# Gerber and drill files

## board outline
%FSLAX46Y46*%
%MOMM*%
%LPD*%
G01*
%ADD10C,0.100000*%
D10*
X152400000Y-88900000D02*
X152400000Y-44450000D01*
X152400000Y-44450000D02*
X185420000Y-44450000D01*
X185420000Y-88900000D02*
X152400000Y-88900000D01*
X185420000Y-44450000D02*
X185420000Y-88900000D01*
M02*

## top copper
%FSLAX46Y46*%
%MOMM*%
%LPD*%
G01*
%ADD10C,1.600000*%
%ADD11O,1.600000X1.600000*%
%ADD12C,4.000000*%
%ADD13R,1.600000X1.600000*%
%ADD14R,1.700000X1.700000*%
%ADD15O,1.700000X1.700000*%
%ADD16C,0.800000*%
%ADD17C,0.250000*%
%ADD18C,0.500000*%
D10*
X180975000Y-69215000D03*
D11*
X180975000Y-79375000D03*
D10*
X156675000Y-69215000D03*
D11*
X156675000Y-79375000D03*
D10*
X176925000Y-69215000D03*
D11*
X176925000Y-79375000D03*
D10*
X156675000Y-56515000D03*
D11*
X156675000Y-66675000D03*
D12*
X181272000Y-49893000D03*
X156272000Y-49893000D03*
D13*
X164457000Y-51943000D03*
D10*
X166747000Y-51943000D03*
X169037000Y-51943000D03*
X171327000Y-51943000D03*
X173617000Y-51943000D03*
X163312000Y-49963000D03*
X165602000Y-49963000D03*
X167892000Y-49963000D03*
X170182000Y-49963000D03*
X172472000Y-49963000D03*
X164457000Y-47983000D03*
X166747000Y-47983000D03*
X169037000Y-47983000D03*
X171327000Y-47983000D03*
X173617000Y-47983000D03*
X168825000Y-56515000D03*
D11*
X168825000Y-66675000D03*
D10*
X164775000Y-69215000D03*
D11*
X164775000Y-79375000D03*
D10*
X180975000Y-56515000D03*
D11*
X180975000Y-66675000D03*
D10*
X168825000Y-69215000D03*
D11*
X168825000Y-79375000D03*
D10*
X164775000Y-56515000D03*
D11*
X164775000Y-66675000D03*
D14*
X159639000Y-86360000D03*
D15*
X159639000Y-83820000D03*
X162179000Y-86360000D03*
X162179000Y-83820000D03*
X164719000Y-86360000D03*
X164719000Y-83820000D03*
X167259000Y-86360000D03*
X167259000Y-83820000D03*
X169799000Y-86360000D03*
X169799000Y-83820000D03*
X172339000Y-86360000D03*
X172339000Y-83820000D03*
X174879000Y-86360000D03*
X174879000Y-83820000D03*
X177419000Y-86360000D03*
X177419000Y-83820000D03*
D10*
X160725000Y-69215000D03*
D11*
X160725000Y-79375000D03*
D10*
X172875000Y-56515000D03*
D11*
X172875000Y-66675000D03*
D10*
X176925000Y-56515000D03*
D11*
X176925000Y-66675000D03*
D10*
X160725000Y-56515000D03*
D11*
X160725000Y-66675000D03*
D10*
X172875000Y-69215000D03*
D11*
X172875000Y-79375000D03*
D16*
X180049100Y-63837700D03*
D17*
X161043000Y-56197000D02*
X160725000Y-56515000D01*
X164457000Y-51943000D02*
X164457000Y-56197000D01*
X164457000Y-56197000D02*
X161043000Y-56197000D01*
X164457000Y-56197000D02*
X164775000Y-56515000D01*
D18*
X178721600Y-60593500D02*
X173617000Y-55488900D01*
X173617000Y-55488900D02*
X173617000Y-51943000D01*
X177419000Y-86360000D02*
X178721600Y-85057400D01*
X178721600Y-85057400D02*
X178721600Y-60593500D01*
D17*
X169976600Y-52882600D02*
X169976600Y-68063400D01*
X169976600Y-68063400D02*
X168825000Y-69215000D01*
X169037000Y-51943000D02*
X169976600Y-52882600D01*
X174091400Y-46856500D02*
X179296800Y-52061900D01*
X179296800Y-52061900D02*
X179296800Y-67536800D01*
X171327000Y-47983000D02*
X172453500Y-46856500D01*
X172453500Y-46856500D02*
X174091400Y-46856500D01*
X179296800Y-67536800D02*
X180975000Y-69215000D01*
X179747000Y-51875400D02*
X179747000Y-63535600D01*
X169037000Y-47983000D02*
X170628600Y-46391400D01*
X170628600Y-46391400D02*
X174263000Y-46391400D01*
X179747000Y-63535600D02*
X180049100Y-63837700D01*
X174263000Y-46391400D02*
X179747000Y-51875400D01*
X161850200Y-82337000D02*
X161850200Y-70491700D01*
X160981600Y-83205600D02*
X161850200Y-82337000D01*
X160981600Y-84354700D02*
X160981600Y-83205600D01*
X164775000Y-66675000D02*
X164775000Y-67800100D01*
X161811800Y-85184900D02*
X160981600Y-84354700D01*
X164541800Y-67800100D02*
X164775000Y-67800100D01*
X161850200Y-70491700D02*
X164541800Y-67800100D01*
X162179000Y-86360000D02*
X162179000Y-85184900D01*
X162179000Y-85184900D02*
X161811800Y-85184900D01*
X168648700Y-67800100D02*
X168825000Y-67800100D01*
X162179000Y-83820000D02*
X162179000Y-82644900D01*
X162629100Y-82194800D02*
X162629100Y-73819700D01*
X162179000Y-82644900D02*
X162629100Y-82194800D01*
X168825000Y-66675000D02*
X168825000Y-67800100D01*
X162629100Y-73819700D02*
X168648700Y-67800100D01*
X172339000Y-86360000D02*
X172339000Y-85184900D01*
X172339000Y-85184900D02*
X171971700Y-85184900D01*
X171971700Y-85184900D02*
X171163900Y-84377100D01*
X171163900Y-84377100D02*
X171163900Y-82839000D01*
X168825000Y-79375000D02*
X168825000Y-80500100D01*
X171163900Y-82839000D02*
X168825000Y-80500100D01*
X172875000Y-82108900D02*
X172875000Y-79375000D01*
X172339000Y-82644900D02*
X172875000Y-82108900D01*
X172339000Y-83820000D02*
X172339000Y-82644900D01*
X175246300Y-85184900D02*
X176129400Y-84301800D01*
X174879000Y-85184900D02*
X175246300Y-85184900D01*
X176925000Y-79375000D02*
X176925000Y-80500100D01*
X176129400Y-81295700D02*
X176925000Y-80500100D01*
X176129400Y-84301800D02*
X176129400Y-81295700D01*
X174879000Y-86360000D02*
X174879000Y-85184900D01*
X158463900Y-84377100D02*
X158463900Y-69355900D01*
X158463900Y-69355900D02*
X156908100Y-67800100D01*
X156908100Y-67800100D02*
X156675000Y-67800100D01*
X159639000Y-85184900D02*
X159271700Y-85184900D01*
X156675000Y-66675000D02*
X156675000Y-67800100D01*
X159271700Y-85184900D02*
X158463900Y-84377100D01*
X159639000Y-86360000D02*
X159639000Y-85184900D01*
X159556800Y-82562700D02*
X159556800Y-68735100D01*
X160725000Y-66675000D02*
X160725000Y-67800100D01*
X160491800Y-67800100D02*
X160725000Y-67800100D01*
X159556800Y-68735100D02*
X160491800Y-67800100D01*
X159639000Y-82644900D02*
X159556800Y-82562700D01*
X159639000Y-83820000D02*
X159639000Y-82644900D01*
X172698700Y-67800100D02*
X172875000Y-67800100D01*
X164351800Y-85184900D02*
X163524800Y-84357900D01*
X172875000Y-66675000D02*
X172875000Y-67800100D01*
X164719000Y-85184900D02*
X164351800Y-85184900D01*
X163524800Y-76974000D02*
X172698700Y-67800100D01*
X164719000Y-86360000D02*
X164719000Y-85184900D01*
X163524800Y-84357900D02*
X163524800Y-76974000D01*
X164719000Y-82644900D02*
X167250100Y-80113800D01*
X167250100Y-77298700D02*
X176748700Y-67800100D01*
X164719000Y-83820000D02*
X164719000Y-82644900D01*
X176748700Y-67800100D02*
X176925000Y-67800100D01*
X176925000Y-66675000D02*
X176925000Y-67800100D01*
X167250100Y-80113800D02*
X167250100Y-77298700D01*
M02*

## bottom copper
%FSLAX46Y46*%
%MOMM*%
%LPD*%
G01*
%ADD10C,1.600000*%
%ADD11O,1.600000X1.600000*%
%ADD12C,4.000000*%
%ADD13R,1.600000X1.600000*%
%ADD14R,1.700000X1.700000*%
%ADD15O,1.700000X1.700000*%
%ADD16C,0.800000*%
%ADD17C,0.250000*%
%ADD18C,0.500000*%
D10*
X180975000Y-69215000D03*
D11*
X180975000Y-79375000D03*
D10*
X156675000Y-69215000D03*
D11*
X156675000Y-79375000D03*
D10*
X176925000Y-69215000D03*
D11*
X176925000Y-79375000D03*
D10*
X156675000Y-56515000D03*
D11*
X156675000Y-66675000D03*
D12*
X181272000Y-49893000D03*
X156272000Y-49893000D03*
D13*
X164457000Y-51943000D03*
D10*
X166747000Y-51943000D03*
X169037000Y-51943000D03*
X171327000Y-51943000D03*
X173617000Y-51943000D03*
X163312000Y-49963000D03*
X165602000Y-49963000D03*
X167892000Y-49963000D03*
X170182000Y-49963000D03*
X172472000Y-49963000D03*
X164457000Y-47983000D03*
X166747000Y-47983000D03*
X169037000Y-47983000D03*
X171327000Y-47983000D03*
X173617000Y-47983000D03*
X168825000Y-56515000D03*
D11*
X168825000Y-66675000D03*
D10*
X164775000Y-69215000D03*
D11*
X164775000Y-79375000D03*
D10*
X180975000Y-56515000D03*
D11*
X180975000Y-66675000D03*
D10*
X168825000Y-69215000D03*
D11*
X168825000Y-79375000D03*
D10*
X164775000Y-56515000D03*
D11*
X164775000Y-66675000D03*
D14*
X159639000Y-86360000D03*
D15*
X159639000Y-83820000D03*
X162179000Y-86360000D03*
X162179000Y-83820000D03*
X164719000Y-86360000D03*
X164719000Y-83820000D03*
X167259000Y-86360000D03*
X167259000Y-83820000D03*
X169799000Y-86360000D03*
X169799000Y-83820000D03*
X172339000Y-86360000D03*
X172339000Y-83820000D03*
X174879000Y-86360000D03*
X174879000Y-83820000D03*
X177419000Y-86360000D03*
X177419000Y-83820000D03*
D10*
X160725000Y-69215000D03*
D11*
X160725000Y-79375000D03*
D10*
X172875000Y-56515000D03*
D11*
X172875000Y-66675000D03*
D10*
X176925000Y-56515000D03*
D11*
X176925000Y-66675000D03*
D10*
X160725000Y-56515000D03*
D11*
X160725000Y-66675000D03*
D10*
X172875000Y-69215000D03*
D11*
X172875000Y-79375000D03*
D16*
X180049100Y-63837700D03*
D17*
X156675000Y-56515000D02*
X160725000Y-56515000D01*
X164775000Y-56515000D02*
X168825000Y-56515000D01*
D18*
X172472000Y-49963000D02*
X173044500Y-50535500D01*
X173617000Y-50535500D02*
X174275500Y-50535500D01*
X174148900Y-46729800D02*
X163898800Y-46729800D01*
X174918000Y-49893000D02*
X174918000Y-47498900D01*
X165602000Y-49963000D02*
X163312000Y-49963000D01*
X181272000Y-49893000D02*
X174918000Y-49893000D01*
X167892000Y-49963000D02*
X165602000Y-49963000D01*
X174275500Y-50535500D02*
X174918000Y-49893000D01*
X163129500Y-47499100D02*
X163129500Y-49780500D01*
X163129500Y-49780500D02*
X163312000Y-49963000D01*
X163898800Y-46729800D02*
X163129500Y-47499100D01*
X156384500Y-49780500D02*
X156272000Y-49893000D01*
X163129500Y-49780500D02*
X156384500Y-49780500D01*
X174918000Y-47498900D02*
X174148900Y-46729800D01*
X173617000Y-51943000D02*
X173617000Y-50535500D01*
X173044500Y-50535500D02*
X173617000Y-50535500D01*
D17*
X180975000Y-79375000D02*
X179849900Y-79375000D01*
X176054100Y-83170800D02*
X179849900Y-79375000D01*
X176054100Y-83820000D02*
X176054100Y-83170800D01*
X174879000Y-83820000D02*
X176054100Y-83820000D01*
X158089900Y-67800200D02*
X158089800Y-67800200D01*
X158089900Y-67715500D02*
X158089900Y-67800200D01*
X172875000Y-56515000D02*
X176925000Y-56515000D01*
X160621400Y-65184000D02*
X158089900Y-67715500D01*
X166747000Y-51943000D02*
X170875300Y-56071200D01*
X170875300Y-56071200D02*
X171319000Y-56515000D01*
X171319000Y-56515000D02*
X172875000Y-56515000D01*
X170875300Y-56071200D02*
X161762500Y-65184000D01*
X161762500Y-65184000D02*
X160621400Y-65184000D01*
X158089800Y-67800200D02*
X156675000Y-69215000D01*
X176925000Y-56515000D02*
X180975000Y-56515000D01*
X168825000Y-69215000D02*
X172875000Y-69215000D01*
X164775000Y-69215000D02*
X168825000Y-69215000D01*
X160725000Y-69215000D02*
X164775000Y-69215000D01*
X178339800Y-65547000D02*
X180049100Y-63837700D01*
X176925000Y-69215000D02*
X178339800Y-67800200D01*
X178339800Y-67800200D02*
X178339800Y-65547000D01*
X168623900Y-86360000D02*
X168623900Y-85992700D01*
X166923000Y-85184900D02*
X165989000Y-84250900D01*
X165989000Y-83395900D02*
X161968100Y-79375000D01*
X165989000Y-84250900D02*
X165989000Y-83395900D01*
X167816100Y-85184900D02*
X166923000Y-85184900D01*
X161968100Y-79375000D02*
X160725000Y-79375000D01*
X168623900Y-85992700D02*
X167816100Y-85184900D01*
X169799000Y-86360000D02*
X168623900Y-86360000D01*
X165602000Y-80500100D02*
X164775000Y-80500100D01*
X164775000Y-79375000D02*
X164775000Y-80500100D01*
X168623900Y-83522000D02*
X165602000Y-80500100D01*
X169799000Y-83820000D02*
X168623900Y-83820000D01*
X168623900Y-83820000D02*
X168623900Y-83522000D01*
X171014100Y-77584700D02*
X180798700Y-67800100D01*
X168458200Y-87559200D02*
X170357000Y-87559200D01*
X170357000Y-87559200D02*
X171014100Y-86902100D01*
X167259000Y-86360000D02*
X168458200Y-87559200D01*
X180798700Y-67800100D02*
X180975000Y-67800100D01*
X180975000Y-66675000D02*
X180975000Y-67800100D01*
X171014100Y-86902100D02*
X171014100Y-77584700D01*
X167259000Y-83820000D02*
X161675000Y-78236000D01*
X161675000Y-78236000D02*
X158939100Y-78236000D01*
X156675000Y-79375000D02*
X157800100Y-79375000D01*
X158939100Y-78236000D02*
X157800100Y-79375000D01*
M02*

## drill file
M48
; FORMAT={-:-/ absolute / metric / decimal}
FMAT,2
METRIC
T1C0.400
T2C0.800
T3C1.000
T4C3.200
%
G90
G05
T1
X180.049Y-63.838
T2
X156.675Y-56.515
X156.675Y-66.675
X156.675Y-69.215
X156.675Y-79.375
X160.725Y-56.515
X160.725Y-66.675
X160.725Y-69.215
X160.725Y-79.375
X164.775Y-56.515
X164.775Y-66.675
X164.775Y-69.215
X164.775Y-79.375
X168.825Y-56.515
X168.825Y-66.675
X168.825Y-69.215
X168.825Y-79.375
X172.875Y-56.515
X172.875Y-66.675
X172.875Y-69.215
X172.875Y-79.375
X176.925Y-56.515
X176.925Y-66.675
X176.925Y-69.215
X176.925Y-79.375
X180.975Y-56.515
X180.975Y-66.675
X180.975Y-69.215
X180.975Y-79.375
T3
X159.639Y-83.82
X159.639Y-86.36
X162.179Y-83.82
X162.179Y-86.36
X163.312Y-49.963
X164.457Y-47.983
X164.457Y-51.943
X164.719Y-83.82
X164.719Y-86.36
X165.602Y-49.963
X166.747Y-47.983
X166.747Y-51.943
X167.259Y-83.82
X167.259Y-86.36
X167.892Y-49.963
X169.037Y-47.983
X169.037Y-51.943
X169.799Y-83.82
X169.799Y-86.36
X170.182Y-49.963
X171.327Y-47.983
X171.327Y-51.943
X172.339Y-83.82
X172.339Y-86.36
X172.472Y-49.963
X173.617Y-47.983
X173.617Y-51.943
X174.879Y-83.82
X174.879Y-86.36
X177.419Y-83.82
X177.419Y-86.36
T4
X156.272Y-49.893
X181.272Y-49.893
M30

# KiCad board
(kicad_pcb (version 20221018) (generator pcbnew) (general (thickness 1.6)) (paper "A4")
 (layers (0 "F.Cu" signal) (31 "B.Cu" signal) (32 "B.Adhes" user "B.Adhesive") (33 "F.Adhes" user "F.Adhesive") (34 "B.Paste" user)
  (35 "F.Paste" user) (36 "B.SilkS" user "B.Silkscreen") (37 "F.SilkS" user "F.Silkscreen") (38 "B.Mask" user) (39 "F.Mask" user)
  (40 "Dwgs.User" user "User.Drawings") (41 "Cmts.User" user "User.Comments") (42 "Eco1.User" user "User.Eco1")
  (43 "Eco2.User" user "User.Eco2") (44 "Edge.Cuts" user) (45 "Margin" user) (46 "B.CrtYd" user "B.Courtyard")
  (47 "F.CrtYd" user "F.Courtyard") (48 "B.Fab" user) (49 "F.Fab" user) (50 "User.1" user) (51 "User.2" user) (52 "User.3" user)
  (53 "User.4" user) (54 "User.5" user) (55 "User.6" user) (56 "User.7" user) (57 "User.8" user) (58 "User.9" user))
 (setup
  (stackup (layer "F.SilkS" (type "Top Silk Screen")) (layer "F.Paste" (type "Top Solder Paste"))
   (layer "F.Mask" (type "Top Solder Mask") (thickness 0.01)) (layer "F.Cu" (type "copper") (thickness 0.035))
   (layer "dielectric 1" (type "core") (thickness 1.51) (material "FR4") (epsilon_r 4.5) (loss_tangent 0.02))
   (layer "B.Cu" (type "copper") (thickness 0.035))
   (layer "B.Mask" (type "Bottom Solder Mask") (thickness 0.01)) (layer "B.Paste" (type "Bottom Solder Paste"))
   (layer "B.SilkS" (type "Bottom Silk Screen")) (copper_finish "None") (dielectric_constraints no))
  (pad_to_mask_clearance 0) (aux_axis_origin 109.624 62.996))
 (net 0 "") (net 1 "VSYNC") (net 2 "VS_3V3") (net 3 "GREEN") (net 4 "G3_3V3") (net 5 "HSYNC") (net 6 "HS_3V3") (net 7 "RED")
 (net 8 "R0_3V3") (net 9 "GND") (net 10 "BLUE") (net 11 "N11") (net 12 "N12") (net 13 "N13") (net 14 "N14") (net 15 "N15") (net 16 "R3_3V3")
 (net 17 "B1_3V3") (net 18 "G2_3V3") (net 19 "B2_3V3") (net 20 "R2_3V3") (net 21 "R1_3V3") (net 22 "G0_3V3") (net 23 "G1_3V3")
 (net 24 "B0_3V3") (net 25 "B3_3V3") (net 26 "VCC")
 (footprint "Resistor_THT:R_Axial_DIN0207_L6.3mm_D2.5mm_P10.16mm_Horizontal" (layer "F.Cu") (at 180.975 69.215 -90)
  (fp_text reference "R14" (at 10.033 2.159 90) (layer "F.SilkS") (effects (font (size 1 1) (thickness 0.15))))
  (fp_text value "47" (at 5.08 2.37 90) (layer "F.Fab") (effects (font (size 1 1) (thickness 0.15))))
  (pad "1" thru_hole circle (at 0 0 270) (size 1.6 1.6) (drill 0.8) (layers "*.Cu" "*.Mask") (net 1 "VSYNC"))
  (pad "2" thru_hole oval (at 10.16 0 270) (size 1.6 1.6) (drill 0.8) (layers "*.Cu" "*.Mask") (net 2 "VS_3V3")))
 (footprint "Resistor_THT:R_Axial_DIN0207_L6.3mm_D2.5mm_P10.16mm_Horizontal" (layer "F.Cu") (at 156.675 69.215 -90)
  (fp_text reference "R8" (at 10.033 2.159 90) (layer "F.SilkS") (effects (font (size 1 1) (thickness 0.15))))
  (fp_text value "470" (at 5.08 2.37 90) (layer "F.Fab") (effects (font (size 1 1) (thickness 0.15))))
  (pad "1" thru_hole circle (at 0 0 270) (size 1.6 1.6) (drill 0.8) (layers "*.Cu" "*.Mask") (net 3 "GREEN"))
  (pad "2" thru_hole oval (at 10.16 0 270) (size 1.6 1.6) (drill 0.8) (layers "*.Cu" "*.Mask") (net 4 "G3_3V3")))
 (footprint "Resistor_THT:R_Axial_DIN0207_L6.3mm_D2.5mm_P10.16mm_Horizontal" (layer "F.Cu") (at 176.925 69.215 -90)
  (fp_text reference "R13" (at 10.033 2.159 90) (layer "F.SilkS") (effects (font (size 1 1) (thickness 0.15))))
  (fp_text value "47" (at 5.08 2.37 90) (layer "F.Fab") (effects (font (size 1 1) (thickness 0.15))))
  (pad "1" thru_hole circle (at 0 0 270) (size 1.6 1.6) (drill 0.8) (layers "*.Cu" "*.Mask") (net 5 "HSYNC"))
  (pad "2" thru_hole oval (at 10.16 0 270) (size 1.6 1.6) (drill 0.8) (layers "*.Cu" "*.Mask") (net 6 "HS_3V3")))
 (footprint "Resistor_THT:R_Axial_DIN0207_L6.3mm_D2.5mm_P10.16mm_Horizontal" (layer "F.Cu") (at 156.675 56.515 -90)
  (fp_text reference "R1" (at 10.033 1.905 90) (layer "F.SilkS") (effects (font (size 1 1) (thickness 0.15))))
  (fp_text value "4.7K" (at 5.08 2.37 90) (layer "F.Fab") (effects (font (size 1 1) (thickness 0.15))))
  (pad "1" thru_hole circle (at 0 0 270) (size 1.6 1.6) (drill 0.8) (layers "*.Cu" "*.Mask") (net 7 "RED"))
  (pad "2" thru_hole oval (at 10.16 0 270) (size 1.6 1.6) (drill 0.8) (layers "*.Cu" "*.Mask") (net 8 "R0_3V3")))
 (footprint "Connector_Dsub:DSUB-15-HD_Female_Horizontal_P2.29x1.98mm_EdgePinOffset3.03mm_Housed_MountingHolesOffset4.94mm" (layer "F.Cu")
  (at 164.457 51.943 180)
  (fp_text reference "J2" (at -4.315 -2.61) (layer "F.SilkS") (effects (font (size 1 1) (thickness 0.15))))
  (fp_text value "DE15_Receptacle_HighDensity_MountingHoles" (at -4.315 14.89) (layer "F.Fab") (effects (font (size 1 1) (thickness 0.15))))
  (pad "0" thru_hole circle (at -16.815 2.05 180) (size 4 4) (drill 3.2) (layers "*.Cu" "*.Mask") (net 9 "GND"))
  (pad "0" thru_hole circle (at 8.185 2.05 180) (size 4 4) (drill 3.2) (layers "*.Cu" "*.Mask") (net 9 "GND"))
  (pad "1" thru_hole rect (at 0 0 180) (size 1.6 1.6) (drill 1) (layers "*.Cu" "*.Mask") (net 7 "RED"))
  (pad "2" thru_hole circle (at -2.29 0 180) (size 1.6 1.6) (drill 1) (layers "*.Cu" "*.Mask") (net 3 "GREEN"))
  (pad "3" thru_hole circle (at -4.58 0 180) (size 1.6 1.6) (drill 1) (layers "*.Cu" "*.Mask") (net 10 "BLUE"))
  (pad "4" thru_hole circle (at -6.87 0 180) (size 1.6 1.6) (drill 1) (layers "*.Cu" "*.Mask") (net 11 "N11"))
  (pad "5" thru_hole circle (at -9.16 0 180) (size 1.6 1.6) (drill 1) (layers "*.Cu" "*.Mask") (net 9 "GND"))
  (pad "6" thru_hole circle (at 1.145 1.98 180) (size 1.6 1.6) (drill 1) (layers "*.Cu" "*.Mask") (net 9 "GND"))
  (pad "7" thru_hole circle (at -1.145 1.98 180) (size 1.6 1.6) (drill 1) (layers "*.Cu" "*.Mask") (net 9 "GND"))
  (pad "8" thru_hole circle (at -3.435 1.98 180) (size 1.6 1.6) (drill 1) (layers "*.Cu" "*.Mask") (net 9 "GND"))
  (pad "9" thru_hole circle (at -5.725 1.98 180) (size 1.6 1.6) (drill 1) (layers "*.Cu" "*.Mask") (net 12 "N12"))
  (pad "10" thru_hole circle (at -8.015 1.98 180) (size 1.6 1.6) (drill 1) (layers "*.Cu" "*.Mask") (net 9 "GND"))
  (pad "11" thru_hole circle (at 0 3.96 180) (size 1.6 1.6) (drill 1) (layers "*.Cu" "*.Mask") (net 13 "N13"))
  (pad "12" thru_hole circle (at -2.29 3.96 180) (size 1.6 1.6) (drill 1) (layers "*.Cu" "*.Mask") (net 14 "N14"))
  (pad "13" thru_hole circle (at -4.58 3.96 180) (size 1.6 1.6) (drill 1) (layers "*.Cu" "*.Mask") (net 5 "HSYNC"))
  (pad "14" thru_hole circle (at -6.87 3.96 180) (size 1.6 1.6) (drill 1) (layers "*.Cu" "*.Mask") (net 1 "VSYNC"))
  (pad "15" thru_hole circle (at -9.16 3.96 180) (size 1.6 1.6) (drill 1) (layers "*.Cu" "*.Mask") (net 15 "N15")))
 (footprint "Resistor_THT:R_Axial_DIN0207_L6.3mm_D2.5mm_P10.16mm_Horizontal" (layer "F.Cu") (at 168.825 56.515 -90)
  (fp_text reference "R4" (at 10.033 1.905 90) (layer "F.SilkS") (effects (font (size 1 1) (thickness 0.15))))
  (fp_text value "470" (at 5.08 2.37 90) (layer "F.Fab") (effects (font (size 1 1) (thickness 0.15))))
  (pad "1" thru_hole circle (at 0 0 270) (size 1.6 1.6) (drill 0.8) (layers "*.Cu" "*.Mask") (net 7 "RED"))
  (pad "2" thru_hole oval (at 10.16 0 270) (size 1.6 1.6) (drill 0.8) (layers "*.Cu" "*.Mask") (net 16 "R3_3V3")))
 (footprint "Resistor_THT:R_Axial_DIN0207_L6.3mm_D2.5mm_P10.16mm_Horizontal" (layer "F.Cu") (at 164.775 69.215 -90)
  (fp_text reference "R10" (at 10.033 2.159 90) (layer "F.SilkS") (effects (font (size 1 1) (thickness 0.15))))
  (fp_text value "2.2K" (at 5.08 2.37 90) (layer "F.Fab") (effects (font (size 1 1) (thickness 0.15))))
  (pad "1" thru_hole circle (at 0 0 270) (size 1.6 1.6) (drill 0.8) (layers "*.Cu" "*.Mask") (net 10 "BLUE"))
  (pad "2" thru_hole oval (at 10.16 0 270) (size 1.6 1.6) (drill 0.8) (layers "*.Cu" "*.Mask") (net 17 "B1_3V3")))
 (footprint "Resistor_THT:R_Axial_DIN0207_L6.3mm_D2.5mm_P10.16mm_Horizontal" (layer "F.Cu") (at 180.975 56.515 -90)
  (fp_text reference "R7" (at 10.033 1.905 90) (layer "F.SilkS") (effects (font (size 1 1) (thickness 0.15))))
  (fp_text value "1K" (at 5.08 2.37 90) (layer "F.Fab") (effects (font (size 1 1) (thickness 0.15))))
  (pad "1" thru_hole circle (at 0 0 270) (size 1.6 1.6) (drill 0.8) (layers "*.Cu" "*.Mask") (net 3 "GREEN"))
  (pad "2" thru_hole oval (at 10.16 0 270) (size 1.6 1.6) (drill 0.8) (layers "*.Cu" "*.Mask") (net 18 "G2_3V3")))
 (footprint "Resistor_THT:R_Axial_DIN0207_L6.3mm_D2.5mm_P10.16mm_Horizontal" (layer "F.Cu") (at 168.825 69.215 -90)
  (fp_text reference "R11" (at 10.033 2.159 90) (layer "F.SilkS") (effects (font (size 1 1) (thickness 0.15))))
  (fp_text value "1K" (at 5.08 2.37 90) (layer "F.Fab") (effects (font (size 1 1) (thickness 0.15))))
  (pad "1" thru_hole circle (at 0 0 270) (size 1.6 1.6) (drill 0.8) (layers "*.Cu" "*.Mask") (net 10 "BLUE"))
  (pad "2" thru_hole oval (at 10.16 0 270) (size 1.6 1.6) (drill 0.8) (layers "*.Cu" "*.Mask") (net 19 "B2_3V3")))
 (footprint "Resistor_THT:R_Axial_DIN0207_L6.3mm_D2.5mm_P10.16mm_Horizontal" (layer "F.Cu") (at 164.775 56.515 -90)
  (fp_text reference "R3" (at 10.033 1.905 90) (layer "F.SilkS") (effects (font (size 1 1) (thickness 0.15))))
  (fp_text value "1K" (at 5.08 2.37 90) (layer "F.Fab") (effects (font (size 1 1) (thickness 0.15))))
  (pad "1" thru_hole circle (at 0 0 270) (size 1.6 1.6) (drill 0.8) (layers "*.Cu" "*.Mask") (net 7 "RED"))
  (pad "2" thru_hole oval (at 10.16 0 270) (size 1.6 1.6) (drill 0.8) (layers "*.Cu" "*.Mask") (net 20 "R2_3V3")))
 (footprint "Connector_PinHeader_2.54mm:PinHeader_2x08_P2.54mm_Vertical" (layer "F.Cu") (at 159.639 86.36 90)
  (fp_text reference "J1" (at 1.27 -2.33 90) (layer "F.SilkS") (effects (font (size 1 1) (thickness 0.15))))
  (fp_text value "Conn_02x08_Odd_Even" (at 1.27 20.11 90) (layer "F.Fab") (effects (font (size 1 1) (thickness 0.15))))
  (pad "1" thru_hole rect (at 0 0 90) (size 1.7 1.7) (drill 1) (layers "*.Cu" "*.Mask") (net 8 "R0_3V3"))
  (pad "2" thru_hole oval (at 2.54 0 90) (size 1.7 1.7) (drill 1) (layers "*.Cu" "*.Mask") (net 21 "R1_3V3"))
  (pad "3" thru_hole oval (at 0 2.54 90) (size 1.7 1.7) (drill 1) (layers "*.Cu" "*.Mask") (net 20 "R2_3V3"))
  (pad "4" thru_hole oval (at 2.54 2.54 90) (size 1.7 1.7) (drill 1) (layers "*.Cu" "*.Mask") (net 16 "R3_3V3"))
  (pad "5" thru_hole oval (at 0 5.08 90) (size 1.7 1.7) (drill 1) (layers "*.Cu" "*.Mask") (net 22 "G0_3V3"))
  (pad "6" thru_hole oval (at 2.54 5.08 90) (size 1.7 1.7) (drill 1) (layers "*.Cu" "*.Mask") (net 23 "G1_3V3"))
  (pad "7" thru_hole oval (at 0 7.62 90) (size 1.7 1.7) (drill 1) (layers "*.Cu" "*.Mask") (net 18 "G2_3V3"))
  (pad "8" thru_hole oval (at 2.54 7.62 90) (size 1.7 1.7) (drill 1) (layers "*.Cu" "*.Mask") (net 4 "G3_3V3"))
  (pad "9" thru_hole oval (at 0 10.16 90) (size 1.7 1.7) (drill 1) (layers "*.Cu" "*.Mask") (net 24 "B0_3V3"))
  (pad "10" thru_hole oval (at 2.54 10.16 90) (size 1.7 1.7) (drill 1) (layers "*.Cu" "*.Mask") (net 17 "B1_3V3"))
  (pad "11" thru_hole oval (at 0 12.7 90) (size 1.7 1.7) (drill 1) (layers "*.Cu" "*.Mask") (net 19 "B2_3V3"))
  (pad "12" thru_hole oval (at 2.54 12.7 90) (size 1.7 1.7) (drill 1) (layers "*.Cu" "*.Mask") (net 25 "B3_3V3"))
  (pad "13" thru_hole oval (at 0 15.24 90) (size 1.7 1.7) (drill 1) (layers "*.Cu" "*.Mask") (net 6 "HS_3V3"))
  (pad "14" thru_hole oval (at 2.54 15.24 90) (size 1.7 1.7) (drill 1) (layers "*.Cu" "*.Mask") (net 2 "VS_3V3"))
  (pad "15" thru_hole oval (at 0 17.78 90) (size 1.7 1.7) (drill 1) (layers "*.Cu" "*.Mask") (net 9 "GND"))
  (pad "16" thru_hole oval (at 2.54 17.78 90) (size 1.7 1.7) (drill 1) (layers "*.Cu" "*.Mask") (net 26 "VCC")))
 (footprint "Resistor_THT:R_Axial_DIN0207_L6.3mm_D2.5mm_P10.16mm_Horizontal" (layer "F.Cu") (at 160.725 69.215 -90)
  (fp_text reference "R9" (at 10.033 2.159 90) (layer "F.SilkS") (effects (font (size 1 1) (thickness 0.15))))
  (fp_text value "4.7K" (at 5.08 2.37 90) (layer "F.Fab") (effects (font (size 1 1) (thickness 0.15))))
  (pad "1" thru_hole circle (at 0 0 270) (size 1.6 1.6) (drill 0.8) (layers "*.Cu" "*.Mask") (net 10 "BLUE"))
  (pad "2" thru_hole oval (at 10.16 0 270) (size 1.6 1.6) (drill 0.8) (layers "*.Cu" "*.Mask") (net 24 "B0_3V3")))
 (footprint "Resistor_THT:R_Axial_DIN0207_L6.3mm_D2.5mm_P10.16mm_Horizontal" (layer "F.Cu") (at 172.875 56.515 -90)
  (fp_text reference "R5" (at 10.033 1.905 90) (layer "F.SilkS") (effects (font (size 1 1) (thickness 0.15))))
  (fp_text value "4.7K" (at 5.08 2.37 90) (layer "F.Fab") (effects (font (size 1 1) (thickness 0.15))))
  (pad "1" thru_hole circle (at 0 0 270) (size 1.6 1.6) (drill 0.8) (layers "*.Cu" "*.Mask") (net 3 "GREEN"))
  (pad "2" thru_hole oval (at 10.16 0 270) (size 1.6 1.6) (drill 0.8) (layers "*.Cu" "*.Mask") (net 22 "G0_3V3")))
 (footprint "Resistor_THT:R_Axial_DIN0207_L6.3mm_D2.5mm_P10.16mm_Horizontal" (layer "F.Cu") (at 176.925 56.515 -90)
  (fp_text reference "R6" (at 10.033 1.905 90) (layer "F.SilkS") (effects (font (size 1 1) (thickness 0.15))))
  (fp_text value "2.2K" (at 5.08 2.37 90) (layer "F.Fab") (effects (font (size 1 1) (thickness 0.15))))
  (pad "1" thru_hole circle (at 0 0 270) (size 1.6 1.6) (drill 0.8) (layers "*.Cu" "*.Mask") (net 3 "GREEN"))
  (pad "2" thru_hole oval (at 10.16 0 270) (size 1.6 1.6) (drill 0.8) (layers "*.Cu" "*.Mask") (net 23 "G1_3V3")))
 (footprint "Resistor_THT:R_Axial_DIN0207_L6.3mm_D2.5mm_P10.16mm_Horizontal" (layer "F.Cu") (at 160.725 56.515 -90)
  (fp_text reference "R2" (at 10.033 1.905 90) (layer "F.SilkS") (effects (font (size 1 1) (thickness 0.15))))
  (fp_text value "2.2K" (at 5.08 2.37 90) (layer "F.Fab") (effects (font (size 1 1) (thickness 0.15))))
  (pad "1" thru_hole circle (at 0 0 270) (size 1.6 1.6) (drill 0.8) (layers "*.Cu" "*.Mask") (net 7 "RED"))
  (pad "2" thru_hole oval (at 10.16 0 270) (size 1.6 1.6) (drill 0.8) (layers "*.Cu" "*.Mask") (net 21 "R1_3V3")))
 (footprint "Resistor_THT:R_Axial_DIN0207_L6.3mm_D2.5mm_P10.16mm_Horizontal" (layer "F.Cu") (at 172.875 69.215 -90)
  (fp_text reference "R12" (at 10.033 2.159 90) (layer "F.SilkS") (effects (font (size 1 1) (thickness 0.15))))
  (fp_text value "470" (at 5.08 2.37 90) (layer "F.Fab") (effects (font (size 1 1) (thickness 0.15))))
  (pad "1" thru_hole circle (at 0 0 270) (size 1.6 1.6) (drill 0.8) (layers "*.Cu" "*.Mask") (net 10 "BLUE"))
  (pad "2" thru_hole oval (at 10.16 0 270) (size 1.6 1.6) (drill 0.8) (layers "*.Cu" "*.Mask") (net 25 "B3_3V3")))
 (gr_line (start 152.4 88.9) (end 152.4 44.45) (stroke (width 0.1) (type default)) (layer "Edge.Cuts"))
 (gr_line (start 152.4 44.45) (end 185.42 44.45) (stroke (width 0.1) (type default)) (layer "Edge.Cuts"))
 (gr_line (start 185.42 88.9) (end 152.4 88.9) (stroke (width 0.1) (type default)) (layer "Edge.Cuts"))
 (gr_line (start 185.42 44.45) (end 185.42 88.9) (stroke (width 0.1) (type default)) (layer "Edge.Cuts"))
 (segment (start 161.043 56.197) (end 160.725 56.515) (width 0.25) (layer "F.Cu") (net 7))
 (segment (start 164.457 51.943) (end 164.457 56.197) (width 0.25) (layer "F.Cu") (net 7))
 (segment (start 164.457 56.197) (end 161.043 56.197) (width 0.25) (layer "F.Cu") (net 7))
 (segment (start 164.457 56.197) (end 164.775 56.515) (width 0.25) (layer "F.Cu") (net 7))
 (segment (start 156.675 56.515) (end 160.725 56.515) (width 0.25) (layer "B.Cu") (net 7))
 (segment (start 164.775 56.515) (end 168.825 56.515) (width 0.25) (layer "B.Cu") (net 7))
 (segment (start 178.7216 60.5935) (end 173.617 55.4889) (width 0.5) (layer "F.Cu") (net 9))
 (segment (start 173.617 55.4889) (end 173.617 51.943) (width 0.5) (layer "F.Cu") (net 9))
 (segment (start 177.419 86.36) (end 178.7216 85.0574) (width 0.5) (layer "F.Cu") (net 9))
 (segment (start 178.7216 85.0574) (end 178.7216 60.5935) (width 0.5) (layer "F.Cu") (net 9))
 (segment (start 172.472 49.963) (end 173.0445 50.5355) (width 0.5) (layer "B.Cu") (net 9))
 (segment (start 173.617 50.5355) (end 174.2755 50.5355) (width 0.5) (layer "B.Cu") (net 9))
 (segment (start 174.1489 46.7298) (end 163.8988 46.7298) (width 0.5) (layer "B.Cu") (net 9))
 (segment (start 174.918 49.893) (end 174.918 47.4989) (width 0.5) (layer "B.Cu") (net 9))
 (segment (start 165.602 49.963) (end 163.312 49.963) (width 0.5) (layer "B.Cu") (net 9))
 (segment (start 181.272 49.893) (end 174.918 49.893) (width 0.5) (layer "B.Cu") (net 9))
 (segment (start 167.892 49.963) (end 165.602 49.963) (width 0.5) (layer "B.Cu") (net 9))
 (segment (start 174.2755 50.5355) (end 174.918 49.893) (width 0.5) (layer "B.Cu") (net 9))
 (segment (start 163.1295 47.4991) (end 163.1295 49.7805) (width 0.5) (layer "B.Cu") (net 9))
 (segment (start 163.1295 49.7805) (end 163.312 49.963) (width 0.5) (layer "B.Cu") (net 9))
 (segment (start 163.8988 46.7298) (end 163.1295 47.4991) (width 0.5) (layer "B.Cu") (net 9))
 (segment (start 156.3845 49.7805) (end 156.272 49.893) (width 0.5) (layer "B.Cu") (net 9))
 (segment (start 163.1295 49.7805) (end 156.3845 49.7805) (width 0.5) (layer "B.Cu") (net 9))
 (segment (start 174.918 47.4989) (end 174.1489 46.7298) (width 0.5) (layer "B.Cu") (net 9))
 (segment (start 173.617 51.943) (end 173.617 50.5355) (width 0.5) (layer "B.Cu") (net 9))
 (segment (start 173.0445 50.5355) (end 173.617 50.5355) (width 0.5) (layer "B.Cu") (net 9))
 (segment (start 180.975 79.375) (end 179.8499 79.375) (width 0.25) (layer "B.Cu") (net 2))
 (segment (start 176.0541 83.1708) (end 179.8499 79.375) (width 0.25) (layer "B.Cu") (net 2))
 (segment (start 176.0541 83.82) (end 176.0541 83.1708) (width 0.25) (layer "B.Cu") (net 2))
 (segment (start 174.879 83.82) (end 176.0541 83.82) (width 0.25) (layer "B.Cu") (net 2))
 (segment (start 158.0899 67.8002) (end 158.0898 67.8002) (width 0.25) (layer "B.Cu") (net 3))
 (segment (start 158.0899 67.7155) (end 158.0899 67.8002) (width 0.25) (layer "B.Cu") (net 3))
 (segment (start 172.875 56.515) (end 176.925 56.515) (width 0.25) (layer "B.Cu") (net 3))
 (segment (start 160.6214 65.184) (end 158.0899 67.7155) (width 0.25) (layer "B.Cu") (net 3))
 (segment (start 166.747 51.943) (end 170.8753 56.0712) (width 0.25) (layer "B.Cu") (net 3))
 (segment (start 170.8753 56.0712) (end 171.319 56.515) (width 0.25) (layer "B.Cu") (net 3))
 (segment (start 171.319 56.515) (end 172.875 56.515) (width 0.25) (layer "B.Cu") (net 3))
 (segment (start 170.8753 56.0712) (end 161.7625 65.184) (width 0.25) (layer "B.Cu") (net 3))
 (segment (start 161.7625 65.184) (end 160.6214 65.184) (width 0.25) (layer "B.Cu") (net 3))
 (segment (start 158.0898 67.8002) (end 156.675 69.215) (width 0.25) (layer "B.Cu") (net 3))
 (segment (start 176.925 56.515) (end 180.975 56.515) (width 0.25) (layer "B.Cu") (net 3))
 (segment (start 169.9766 52.8826) (end 169.9766 68.0634) (width 0.25) (layer "F.Cu") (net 10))
 (segment (start 169.9766 68.0634) (end 168.825 69.215) (width 0.25) (layer "F.Cu") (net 10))
 (segment (start 169.037 51.943) (end 169.9766 52.8826) (width 0.25) (layer "F.Cu") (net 10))
 (segment (start 168.825 69.215) (end 172.875 69.215) (width 0.25) (layer "B.Cu") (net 10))
 (segment (start 164.775 69.215) (end 168.825 69.215) (width 0.25) (layer "B.Cu") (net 10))
 (segment (start 160.725 69.215) (end 164.775 69.215) (width 0.25) (layer "B.Cu") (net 10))
 (segment (start 174.0914 46.8565) (end 179.2968 52.0619) (width 0.25) (layer "F.Cu") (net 1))
 (segment (start 179.2968 52.0619) (end 179.2968 67.5368) (width 0.25) (layer "F.Cu") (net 1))
 (segment (start 171.327 47.983) (end 172.4535 46.8565) (width 0.25) (layer "F.Cu") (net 1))
 (segment (start 172.4535 46.8565) (end 174.0914 46.8565) (width 0.25) (layer "F.Cu") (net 1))
 (segment (start 179.2968 67.5368) (end 180.975 69.215) (width 0.25) (layer "F.Cu") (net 1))
 (segment (start 179.747 51.8754) (end 179.747 63.5356) (width 0.25) (layer "F.Cu") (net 5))
 (segment (start 169.037 47.983) (end 170.6286 46.3914) (width 0.25) (layer "F.Cu") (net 5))
 (segment (start 170.6286 46.3914) (end 174.263 46.3914) (width 0.25) (layer "F.Cu") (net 5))
 (segment (start 179.747 63.5356) (end 180.0491 63.8377) (width 0.25) (layer "F.Cu") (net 5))
 (segment (start 174.263 46.3914) (end 179.747 51.8754) (width 0.25) (layer "F.Cu") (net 5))
 (via (at 180.0491 63.8377) (size 0.8) (drill 0.4) (layers "F.Cu" "B.Cu") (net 5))
 (segment (start 178.3398 65.547) (end 180.0491 63.8377) (width 0.25) (layer "B.Cu") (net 5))
 (segment (start 176.925 69.215) (end 178.3398 67.8002) (width 0.25) (layer "B.Cu") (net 5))
 (segment (start 178.3398 67.8002) (end 178.3398 65.547) (width 0.25) (layer "B.Cu") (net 5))
 (segment (start 161.8502 82.337) (end 161.8502 70.4917) (width 0.25) (layer "F.Cu") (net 20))
 (segment (start 160.9816 83.2056) (end 161.8502 82.337) (width 0.25) (layer "F.Cu") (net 20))
 (segment (start 160.9816 84.3547) (end 160.9816 83.2056) (width 0.25) (layer "F.Cu") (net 20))
 (segment (start 164.775 66.675) (end 164.775 67.8001) (width 0.25) (layer "F.Cu") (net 20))
 (segment (start 161.8118 85.1849) (end 160.9816 84.3547) (width 0.25) (layer "F.Cu") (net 20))
 (segment (start 164.5418 67.8001) (end 164.775 67.8001) (width 0.25) (layer "F.Cu") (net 20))
 (segment (start 161.8502 70.4917) (end 164.5418 67.8001) (width 0.25) (layer "F.Cu") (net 20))
 (segment (start 162.179 86.36) (end 162.179 85.1849) (width 0.25) (layer "F.Cu") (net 20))
 (segment (start 162.179 85.1849) (end 161.8118 85.1849) (width 0.25) (layer "F.Cu") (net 20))
 (segment (start 168.6487 67.8001) (end 168.825 67.8001) (width 0.25) (layer "F.Cu") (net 16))
 (segment (start 162.179 83.82) (end 162.179 82.6449) (width 0.25) (layer "F.Cu") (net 16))
 (segment (start 162.6291 82.1948) (end 162.6291 73.8197) (width 0.25) (layer "F.Cu") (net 16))
 (segment (start 162.179 82.6449) (end 162.6291 82.1948) (width 0.25) (layer "F.Cu") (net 16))
 (segment (start 168.825 66.675) (end 168.825 67.8001) (width 0.25) (layer "F.Cu") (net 16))
 (segment (start 162.6291 73.8197) (end 168.6487 67.8001) (width 0.25) (layer "F.Cu") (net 16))
 (segment (start 168.6239 86.36) (end 168.6239 85.9927) (width 0.25) (layer "B.Cu") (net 24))
 (segment (start 166.923 85.1849) (end 165.989 84.2509) (width 0.25) (layer "B.Cu") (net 24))
 (segment (start 165.989 83.3959) (end 161.9681 79.375) (width 0.25) (layer "B.Cu") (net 24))
 (segment (start 165.989 84.2509) (end 165.989 83.3959) (width 0.25) (layer "B.Cu") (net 24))
 (segment (start 167.8161 85.1849) (end 166.923 85.1849) (width 0.25) (layer "B.Cu") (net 24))
 (segment (start 161.9681 79.375) (end 160.725 79.375) (width 0.25) (layer "B.Cu") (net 24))
 (segment (start 168.6239 85.9927) (end 167.8161 85.1849) (width 0.25) (layer "B.Cu") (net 24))
 (segment (start 169.799 86.36) (end 168.6239 86.36) (width 0.25) (layer "B.Cu") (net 24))
 (segment (start 165.602 80.5001) (end 164.775 80.5001) (width 0.25) (layer "B.Cu") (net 17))
 (segment (start 164.775 79.375) (end 164.775 80.5001) (width 0.25) (layer "B.Cu") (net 17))
 (segment (start 168.6239 83.522) (end 165.602 80.5001) (width 0.25) (layer "B.Cu") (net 17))
 (segment (start 169.799 83.82) (end 168.6239 83.82) (width 0.25) (layer "B.Cu") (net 17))
 (segment (start 168.6239 83.82) (end 168.6239 83.522) (width 0.25) (layer "B.Cu") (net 17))
 (segment (start 172.339 86.36) (end 172.339 85.1849) (width 0.25) (layer "F.Cu") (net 19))
 (segment (start 172.339 85.1849) (end 171.9717 85.1849) (width 0.25) (layer "F.Cu") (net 19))
 (segment (start 171.9717 85.1849) (end 171.1639 84.3771) (width 0.25) (layer "F.Cu") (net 19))
 (segment (start 171.1639 84.3771) (end 171.1639 82.839) (width 0.25) (layer "F.Cu") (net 19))
 (segment (start 168.825 79.375) (end 168.825 80.5001) (width 0.25) (layer "F.Cu") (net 19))
 (segment (start 171.1639 82.839) (end 168.825 80.5001) (width 0.25) (layer "F.Cu") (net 19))
 (segment (start 172.875 82.1089) (end 172.875 79.375) (width 0.25) (layer "F.Cu") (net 25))
 (segment (start 172.339 82.6449) (end 172.875 82.1089) (width 0.25) (layer "F.Cu") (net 25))
 (segment (start 172.339 83.82) (end 172.339 82.6449) (width 0.25) (layer "F.Cu") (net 25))
 (segment (start 175.2463 85.1849) (end 176.1294 84.3018) (width 0.25) (layer "F.Cu") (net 6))
 (segment (start 174.879 85.1849) (end 175.2463 85.1849) (width 0.25) (layer "F.Cu") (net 6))
 (segment (start 176.925 79.375) (end 176.925 80.5001) (width 0.25) (layer "F.Cu") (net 6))
 (segment (start 176.1294 81.2957) (end 176.925 80.5001) (width 0.25) (layer "F.Cu") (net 6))
 (segment (start 176.1294 84.3018) (end 176.1294 81.2957) (width 0.25) (layer "F.Cu") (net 6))
 (segment (start 174.879 86.36) (end 174.879 85.1849) (width 0.25) (layer "F.Cu") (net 6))
 (segment (start 158.4639 84.3771) (end 158.4639 69.3559) (width 0.25) (layer "F.Cu") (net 8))
 (segment (start 158.4639 69.3559) (end 156.9081 67.8001) (width 0.25) (layer "F.Cu") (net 8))
 (segment (start 156.9081 67.8001) (end 156.675 67.8001) (width 0.25) (layer "F.Cu") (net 8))
 (segment (start 159.639 85.1849) (end 159.2717 85.1849) (width 0.25) (layer "F.Cu") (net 8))
 (segment (start 156.675 66.675) (end 156.675 67.8001) (width 0.25) (layer "F.Cu") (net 8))
 (segment (start 159.2717 85.1849) (end 158.4639 84.3771) (width 0.25) (layer "F.Cu") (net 8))
 (segment (start 159.639 86.36) (end 159.639 85.1849) (width 0.25) (layer "F.Cu") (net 8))
 (segment (start 159.5568 82.5627) (end 159.5568 68.7351) (width 0.25) (layer "F.Cu") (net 21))
 (segment (start 160.725 66.675) (end 160.725 67.8001) (width 0.25) (layer "F.Cu") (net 21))
 (segment (start 160.4918 67.8001) (end 160.725 67.8001) (width 0.25) (layer "F.Cu") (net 21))
 (segment (start 159.5568 68.7351) (end 160.4918 67.8001) (width 0.25) (layer "F.Cu") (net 21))
 (segment (start 159.639 82.6449) (end 159.5568 82.5627) (width 0.25) (layer "F.Cu") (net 21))
 (segment (start 159.639 83.82) (end 159.639 82.6449) (width 0.25) (layer "F.Cu") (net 21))
 (segment (start 172.6987 67.8001) (end 172.875 67.8001) (width 0.25) (layer "F.Cu") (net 22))
 (segment (start 164.3518 85.1849) (end 163.5248 84.3579) (width 0.25) (layer "F.Cu") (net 22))
 (segment (start 172.875 66.675) (end 172.875 67.8001) (width 0.25) (layer "F.Cu") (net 22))
 (segment (start 164.719 85.1849) (end 164.3518 85.1849) (width 0.25) (layer "F.Cu") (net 22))
 (segment (start 163.5248 76.974) (end 172.6987 67.8001) (width 0.25) (layer "F.Cu") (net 22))
 (segment (start 164.719 86.36) (end 164.719 85.1849) (width 0.25) (layer "F.Cu") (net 22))
 (segment (start 163.5248 84.3579) (end 163.5248 76.974) (width 0.25) (layer "F.Cu") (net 22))
 (segment (start 164.719 82.6449) (end 167.2501 80.1138) (width 0.25) (layer "F.Cu") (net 23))
 (segment (start 167.2501 77.2987) (end 176.7487 67.8001) (width 0.25) (layer "F.Cu") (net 23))
 (segment (start 164.719 83.82) (end 164.719 82.6449) (width 0.25) (layer "F.Cu") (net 23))
 (segment (start 176.7487 67.8001) (end 176.925 67.8001) (width 0.25) (layer "F.Cu") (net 23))
 (segment (start 176.925 66.675) (end 176.925 67.8001) (width 0.25) (layer "F.Cu") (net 23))
 (segment (start 167.2501 80.1138) (end 167.2501 77.2987) (width 0.25) (layer "F.Cu") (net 23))
 (segment (start 171.0141 77.5847) (end 180.7987 67.8001) (width 0.25) (layer "B.Cu") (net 18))
 (segment (start 168.4582 87.5592) (end 170.357 87.5592) (width 0.25) (layer "B.Cu") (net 18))
 (segment (start 170.357 87.5592) (end 171.0141 86.9021) (width 0.25) (layer "B.Cu") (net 18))
 (segment (start 167.259 86.36) (end 168.4582 87.5592) (width 0.25) (layer "B.Cu") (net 18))
 (segment (start 180.7987 67.8001) (end 180.975 67.8001) (width 0.25) (layer "B.Cu") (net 18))
 (segment (start 180.975 66.675) (end 180.975 67.8001) (width 0.25) (layer "B.Cu") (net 18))
 (segment (start 171.0141 86.9021) (end 171.0141 77.5847) (width 0.25) (layer "B.Cu") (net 18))
 (segment (start 167.259 83.82) (end 161.675 78.236) (width 0.25) (layer "B.Cu") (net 4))
 (segment (start 161.675 78.236) (end 158.9391 78.236) (width 0.25) (layer "B.Cu") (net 4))
 (segment (start 156.675 79.375) (end 157.8001 79.375) (width 0.25) (layer "B.Cu") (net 4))
 (segment (start 158.9391 78.236) (end 157.8001 79.375) (width 0.25) (layer "B.Cu") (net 4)))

